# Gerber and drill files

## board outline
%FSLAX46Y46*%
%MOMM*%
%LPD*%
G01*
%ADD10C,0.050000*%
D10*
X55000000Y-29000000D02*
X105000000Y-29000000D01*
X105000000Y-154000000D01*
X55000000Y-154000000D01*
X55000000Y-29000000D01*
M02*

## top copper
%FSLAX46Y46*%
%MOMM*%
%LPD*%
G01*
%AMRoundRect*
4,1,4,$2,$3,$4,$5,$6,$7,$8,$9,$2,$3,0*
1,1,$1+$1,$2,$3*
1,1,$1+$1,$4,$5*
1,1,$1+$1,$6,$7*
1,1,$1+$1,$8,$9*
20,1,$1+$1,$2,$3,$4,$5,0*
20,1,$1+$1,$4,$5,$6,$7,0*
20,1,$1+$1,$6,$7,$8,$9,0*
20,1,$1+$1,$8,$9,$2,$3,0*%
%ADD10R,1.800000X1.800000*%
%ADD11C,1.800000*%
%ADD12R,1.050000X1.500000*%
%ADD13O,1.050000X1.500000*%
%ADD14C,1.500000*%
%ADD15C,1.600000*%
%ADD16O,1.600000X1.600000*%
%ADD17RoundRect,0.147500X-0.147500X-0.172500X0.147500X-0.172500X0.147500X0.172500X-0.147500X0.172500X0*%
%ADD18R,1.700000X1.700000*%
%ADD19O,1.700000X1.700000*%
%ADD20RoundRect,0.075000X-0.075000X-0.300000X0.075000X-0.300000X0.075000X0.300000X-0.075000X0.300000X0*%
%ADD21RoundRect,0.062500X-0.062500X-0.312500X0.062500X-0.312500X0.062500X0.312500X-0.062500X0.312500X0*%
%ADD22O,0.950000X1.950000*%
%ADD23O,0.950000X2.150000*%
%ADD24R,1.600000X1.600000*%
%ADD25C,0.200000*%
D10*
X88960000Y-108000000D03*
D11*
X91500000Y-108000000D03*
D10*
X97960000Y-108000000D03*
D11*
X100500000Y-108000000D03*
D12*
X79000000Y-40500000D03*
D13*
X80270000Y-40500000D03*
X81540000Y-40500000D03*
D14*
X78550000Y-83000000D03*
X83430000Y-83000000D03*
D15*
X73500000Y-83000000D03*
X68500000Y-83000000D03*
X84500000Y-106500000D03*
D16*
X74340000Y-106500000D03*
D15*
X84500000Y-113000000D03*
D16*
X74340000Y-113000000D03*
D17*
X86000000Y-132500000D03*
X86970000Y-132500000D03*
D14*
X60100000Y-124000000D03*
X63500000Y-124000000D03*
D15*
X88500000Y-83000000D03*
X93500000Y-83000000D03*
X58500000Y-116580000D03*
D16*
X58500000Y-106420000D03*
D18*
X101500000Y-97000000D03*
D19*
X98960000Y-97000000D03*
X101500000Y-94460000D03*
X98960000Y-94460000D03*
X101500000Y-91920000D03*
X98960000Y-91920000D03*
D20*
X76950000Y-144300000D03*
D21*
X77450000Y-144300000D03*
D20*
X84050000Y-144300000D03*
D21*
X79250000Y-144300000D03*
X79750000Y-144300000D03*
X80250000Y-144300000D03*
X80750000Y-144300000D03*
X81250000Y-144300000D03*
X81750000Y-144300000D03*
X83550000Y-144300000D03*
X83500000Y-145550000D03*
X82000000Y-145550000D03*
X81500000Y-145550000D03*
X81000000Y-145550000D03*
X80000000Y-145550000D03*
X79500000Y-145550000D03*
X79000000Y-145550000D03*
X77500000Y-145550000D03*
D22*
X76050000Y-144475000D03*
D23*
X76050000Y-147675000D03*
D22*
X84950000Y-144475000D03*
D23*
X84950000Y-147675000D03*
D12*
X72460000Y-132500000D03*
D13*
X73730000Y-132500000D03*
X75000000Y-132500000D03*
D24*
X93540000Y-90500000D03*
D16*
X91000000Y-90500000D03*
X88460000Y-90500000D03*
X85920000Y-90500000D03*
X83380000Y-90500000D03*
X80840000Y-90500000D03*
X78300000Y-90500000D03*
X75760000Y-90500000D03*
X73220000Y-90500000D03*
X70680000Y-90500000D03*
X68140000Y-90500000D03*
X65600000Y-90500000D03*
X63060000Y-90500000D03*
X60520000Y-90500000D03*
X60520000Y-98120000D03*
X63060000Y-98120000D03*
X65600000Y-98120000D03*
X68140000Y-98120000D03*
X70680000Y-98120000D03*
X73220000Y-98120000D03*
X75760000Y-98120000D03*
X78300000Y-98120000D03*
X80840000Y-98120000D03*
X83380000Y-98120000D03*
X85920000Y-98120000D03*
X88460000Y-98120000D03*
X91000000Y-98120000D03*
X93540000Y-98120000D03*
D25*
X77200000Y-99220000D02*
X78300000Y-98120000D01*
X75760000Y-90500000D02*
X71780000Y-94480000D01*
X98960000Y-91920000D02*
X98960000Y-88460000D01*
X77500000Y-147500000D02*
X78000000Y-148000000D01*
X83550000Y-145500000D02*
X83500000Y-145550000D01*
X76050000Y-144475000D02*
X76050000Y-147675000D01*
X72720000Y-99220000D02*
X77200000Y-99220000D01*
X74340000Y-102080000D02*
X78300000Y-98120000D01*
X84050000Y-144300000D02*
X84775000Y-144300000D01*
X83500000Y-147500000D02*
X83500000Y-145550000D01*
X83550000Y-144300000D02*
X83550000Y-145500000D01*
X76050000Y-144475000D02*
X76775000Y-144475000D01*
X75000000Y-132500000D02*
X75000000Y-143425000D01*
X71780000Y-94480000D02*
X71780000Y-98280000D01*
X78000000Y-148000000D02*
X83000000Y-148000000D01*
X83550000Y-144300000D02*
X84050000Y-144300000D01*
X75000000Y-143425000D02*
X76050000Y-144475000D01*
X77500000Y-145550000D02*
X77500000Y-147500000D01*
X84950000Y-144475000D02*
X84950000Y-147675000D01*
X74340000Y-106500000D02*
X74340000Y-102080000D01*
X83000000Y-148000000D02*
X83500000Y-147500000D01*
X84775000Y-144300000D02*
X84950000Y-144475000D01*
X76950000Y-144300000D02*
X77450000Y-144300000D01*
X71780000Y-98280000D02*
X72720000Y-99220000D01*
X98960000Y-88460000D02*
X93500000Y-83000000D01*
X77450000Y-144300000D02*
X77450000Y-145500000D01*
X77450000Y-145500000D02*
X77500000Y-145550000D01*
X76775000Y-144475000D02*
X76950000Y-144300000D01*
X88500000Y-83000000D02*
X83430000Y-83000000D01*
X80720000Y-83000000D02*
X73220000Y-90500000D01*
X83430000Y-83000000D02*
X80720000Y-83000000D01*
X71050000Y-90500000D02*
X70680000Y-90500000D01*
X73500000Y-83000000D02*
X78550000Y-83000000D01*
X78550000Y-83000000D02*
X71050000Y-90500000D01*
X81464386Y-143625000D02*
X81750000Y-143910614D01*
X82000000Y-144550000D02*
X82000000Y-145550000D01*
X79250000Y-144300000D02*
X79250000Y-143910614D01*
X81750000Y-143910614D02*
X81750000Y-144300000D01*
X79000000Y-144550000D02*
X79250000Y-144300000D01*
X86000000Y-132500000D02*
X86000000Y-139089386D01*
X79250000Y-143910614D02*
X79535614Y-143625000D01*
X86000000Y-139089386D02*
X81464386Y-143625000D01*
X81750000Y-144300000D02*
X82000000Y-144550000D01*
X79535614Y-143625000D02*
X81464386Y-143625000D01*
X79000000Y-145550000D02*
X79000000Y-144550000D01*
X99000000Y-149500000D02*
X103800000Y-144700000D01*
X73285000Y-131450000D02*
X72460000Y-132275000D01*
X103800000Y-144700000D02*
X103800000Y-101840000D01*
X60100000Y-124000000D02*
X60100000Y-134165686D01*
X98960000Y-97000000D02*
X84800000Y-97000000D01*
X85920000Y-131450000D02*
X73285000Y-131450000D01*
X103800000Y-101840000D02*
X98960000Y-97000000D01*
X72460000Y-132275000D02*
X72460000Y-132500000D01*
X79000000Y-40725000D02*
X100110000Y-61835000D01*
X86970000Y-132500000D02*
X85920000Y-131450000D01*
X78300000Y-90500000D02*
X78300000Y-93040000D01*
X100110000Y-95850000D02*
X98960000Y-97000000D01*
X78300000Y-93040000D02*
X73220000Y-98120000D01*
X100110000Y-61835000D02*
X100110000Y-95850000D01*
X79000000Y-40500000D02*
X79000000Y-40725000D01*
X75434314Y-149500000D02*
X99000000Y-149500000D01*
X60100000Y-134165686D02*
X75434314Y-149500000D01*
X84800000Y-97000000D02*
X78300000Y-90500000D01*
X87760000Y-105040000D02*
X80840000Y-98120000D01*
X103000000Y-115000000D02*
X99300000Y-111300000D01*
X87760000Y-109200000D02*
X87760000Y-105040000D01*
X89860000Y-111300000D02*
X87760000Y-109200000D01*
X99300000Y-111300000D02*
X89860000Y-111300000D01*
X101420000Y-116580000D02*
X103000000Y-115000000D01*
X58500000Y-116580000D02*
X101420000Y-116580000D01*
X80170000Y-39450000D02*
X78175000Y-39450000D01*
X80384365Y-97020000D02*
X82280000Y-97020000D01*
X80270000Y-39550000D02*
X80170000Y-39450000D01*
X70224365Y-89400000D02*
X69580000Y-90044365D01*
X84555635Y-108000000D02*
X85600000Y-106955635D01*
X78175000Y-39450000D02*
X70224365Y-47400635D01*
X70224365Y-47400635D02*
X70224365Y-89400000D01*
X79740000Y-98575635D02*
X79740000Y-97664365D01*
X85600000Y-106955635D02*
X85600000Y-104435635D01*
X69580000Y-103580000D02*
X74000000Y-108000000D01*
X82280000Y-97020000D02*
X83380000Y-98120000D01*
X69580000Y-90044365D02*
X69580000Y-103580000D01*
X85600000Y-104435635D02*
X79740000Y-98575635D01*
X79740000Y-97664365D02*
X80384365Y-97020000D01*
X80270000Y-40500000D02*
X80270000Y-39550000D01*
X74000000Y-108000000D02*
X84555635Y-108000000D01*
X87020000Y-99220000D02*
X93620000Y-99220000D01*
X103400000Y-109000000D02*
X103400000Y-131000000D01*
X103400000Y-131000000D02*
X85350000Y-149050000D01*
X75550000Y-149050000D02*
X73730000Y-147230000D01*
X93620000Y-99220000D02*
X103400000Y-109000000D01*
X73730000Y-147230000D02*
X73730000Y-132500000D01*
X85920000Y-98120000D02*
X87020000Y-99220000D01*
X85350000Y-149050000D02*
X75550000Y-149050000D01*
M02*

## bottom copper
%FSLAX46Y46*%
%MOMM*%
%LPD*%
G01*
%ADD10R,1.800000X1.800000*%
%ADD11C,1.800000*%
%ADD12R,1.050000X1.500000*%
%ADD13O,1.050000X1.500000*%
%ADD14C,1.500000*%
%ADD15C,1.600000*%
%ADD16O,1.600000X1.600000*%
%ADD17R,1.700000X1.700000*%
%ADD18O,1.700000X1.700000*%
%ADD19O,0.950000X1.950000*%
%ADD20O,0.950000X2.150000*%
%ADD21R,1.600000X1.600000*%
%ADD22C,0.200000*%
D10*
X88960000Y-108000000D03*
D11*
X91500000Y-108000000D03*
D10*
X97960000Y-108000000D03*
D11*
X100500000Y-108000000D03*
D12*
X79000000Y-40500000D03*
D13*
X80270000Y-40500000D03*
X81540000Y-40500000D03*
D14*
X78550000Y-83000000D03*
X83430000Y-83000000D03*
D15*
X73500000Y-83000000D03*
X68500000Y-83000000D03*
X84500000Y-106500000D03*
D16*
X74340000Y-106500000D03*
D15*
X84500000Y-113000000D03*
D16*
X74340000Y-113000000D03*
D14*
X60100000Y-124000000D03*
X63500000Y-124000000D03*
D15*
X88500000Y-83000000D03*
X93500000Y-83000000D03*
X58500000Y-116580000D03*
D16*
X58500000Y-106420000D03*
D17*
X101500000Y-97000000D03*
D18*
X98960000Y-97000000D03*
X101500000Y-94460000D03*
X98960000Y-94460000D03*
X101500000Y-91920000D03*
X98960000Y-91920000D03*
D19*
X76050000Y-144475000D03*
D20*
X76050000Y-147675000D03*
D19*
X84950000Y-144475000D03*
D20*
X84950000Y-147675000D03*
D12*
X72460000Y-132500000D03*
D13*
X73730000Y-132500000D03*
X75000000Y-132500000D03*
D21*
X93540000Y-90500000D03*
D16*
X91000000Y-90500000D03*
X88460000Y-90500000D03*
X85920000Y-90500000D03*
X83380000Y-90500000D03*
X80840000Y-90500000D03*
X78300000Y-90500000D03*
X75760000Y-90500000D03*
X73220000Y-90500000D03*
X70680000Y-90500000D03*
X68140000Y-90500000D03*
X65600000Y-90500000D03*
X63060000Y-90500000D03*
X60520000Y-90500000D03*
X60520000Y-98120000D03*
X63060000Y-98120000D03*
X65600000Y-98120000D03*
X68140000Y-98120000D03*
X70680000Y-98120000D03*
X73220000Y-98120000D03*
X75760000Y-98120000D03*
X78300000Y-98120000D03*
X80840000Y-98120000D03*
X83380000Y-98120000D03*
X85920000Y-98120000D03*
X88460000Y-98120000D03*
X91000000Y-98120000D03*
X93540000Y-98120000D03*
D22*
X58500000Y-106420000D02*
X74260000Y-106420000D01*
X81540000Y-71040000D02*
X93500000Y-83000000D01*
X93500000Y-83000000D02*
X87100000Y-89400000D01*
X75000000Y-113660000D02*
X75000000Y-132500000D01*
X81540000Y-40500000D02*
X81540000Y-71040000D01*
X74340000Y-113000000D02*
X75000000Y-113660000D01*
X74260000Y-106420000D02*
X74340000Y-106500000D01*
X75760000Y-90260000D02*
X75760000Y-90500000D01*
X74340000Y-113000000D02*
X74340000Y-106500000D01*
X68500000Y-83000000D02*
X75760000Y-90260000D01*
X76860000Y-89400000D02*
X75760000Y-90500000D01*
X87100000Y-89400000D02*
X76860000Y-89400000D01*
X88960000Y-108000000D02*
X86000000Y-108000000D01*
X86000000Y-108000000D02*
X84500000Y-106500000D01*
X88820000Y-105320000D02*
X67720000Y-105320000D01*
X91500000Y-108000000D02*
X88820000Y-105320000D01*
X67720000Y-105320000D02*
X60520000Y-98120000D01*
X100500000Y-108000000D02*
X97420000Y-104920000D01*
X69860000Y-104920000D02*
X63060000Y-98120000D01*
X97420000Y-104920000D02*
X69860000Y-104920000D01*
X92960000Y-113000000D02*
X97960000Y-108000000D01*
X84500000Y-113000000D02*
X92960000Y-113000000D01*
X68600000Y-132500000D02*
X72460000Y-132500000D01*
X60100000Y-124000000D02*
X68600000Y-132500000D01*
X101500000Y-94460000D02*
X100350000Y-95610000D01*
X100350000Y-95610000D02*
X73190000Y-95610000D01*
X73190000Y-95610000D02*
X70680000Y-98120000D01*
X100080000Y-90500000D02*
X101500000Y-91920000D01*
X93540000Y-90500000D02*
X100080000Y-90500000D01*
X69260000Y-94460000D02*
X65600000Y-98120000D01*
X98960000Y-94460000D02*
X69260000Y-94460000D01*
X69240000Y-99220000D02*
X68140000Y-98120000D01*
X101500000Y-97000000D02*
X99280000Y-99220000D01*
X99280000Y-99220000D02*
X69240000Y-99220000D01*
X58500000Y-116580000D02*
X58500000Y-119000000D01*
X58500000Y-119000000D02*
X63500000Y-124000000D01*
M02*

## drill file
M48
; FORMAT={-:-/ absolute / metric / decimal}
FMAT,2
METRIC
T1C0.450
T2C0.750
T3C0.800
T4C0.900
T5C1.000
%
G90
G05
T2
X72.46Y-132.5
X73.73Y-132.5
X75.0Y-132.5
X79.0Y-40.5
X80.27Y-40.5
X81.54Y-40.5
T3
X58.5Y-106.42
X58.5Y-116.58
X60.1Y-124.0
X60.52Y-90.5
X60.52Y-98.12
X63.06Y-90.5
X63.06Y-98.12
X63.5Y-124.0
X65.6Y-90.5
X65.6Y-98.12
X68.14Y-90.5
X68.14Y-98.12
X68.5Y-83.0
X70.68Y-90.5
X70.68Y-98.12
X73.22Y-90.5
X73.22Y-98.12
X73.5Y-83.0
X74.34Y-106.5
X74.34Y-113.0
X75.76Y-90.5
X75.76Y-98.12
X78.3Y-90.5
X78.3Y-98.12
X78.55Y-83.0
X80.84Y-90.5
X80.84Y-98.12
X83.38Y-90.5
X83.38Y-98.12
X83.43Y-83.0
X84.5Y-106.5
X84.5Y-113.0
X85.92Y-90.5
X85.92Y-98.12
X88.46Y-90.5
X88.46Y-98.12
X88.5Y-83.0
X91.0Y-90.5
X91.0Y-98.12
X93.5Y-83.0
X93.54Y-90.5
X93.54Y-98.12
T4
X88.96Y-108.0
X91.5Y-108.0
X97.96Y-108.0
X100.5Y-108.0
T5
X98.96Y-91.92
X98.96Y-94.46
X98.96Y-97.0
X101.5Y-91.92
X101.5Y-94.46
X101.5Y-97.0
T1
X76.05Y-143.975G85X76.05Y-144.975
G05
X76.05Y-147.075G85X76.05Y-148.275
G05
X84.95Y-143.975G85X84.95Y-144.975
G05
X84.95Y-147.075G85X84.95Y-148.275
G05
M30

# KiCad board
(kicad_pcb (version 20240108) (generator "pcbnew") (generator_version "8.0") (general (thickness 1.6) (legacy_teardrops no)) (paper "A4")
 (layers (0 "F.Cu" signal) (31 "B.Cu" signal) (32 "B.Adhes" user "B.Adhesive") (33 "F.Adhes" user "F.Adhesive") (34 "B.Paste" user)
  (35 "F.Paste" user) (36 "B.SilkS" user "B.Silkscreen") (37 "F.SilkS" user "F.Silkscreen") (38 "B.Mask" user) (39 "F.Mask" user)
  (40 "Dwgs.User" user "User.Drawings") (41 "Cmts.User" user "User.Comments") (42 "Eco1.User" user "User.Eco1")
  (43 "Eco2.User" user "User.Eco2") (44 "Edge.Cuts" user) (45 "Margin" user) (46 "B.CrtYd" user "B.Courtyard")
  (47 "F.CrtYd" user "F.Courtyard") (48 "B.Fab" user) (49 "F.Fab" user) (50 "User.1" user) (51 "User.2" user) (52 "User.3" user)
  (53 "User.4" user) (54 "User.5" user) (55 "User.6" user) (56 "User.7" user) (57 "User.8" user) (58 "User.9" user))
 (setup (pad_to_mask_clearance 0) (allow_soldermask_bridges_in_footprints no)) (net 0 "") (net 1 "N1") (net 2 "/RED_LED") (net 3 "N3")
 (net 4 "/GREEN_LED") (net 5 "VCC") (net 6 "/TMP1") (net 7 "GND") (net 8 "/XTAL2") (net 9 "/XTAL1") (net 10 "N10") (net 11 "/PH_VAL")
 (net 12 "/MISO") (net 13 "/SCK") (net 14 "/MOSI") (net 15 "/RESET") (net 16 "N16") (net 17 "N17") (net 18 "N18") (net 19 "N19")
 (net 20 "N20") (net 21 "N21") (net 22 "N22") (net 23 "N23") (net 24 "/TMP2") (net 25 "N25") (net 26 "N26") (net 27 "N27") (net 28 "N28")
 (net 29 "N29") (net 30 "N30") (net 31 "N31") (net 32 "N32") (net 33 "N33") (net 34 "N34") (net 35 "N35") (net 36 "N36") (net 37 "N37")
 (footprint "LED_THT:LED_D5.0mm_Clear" (layer "F.Cu") (at 88.96 108)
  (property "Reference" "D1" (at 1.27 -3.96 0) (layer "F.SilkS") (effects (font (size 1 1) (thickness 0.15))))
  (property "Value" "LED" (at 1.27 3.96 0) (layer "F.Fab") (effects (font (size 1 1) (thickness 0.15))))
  (pad "1" thru_hole rect (at 0 0) (size 1.8 1.8) (drill 0.9) (layers "*.Cu" "*.Mask") (remove_unused_layers no) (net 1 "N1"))
  (pad "2" thru_hole circle (at 2.54 0) (size 1.8 1.8) (drill 0.9) (layers "*.Cu" "*.Mask") (remove_unused_layers no) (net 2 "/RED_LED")))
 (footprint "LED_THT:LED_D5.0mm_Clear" (layer "F.Cu") (at 97.96 108)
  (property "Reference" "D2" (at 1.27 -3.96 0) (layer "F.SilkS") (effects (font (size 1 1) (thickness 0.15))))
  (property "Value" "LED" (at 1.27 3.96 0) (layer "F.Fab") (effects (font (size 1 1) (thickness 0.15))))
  (pad "1" thru_hole rect (at 0 0) (size 1.8 1.8) (drill 0.9) (layers "*.Cu" "*.Mask") (remove_unused_layers no) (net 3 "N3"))
  (pad "2" thru_hole circle (at 2.54 0) (size 1.8 1.8) (drill 0.9) (layers "*.Cu" "*.Mask") (remove_unused_layers no) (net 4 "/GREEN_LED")))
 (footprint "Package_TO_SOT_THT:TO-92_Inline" (layer "F.Cu") (at 79 40.5)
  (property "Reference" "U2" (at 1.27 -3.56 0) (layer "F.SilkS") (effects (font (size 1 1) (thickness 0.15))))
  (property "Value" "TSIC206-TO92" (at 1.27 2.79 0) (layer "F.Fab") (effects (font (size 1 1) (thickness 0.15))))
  (pad "1" thru_hole rect (at 0 0) (size 1.05 1.5) (drill 0.75) (layers "*.Cu" "*.Mask") (remove_unused_layers no) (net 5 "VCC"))
  (pad "2" thru_hole oval (at 1.27 0) (size 1.05 1.5) (drill 0.75) (layers "*.Cu" "*.Mask") (remove_unused_layers no) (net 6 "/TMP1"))
  (pad "3" thru_hole oval (at 2.54 0) (size 1.05 1.5) (drill 0.75) (layers "*.Cu" "*.Mask") (remove_unused_layers no) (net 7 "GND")))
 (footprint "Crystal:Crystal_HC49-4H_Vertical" (layer "F.Cu") (at 78.55 83)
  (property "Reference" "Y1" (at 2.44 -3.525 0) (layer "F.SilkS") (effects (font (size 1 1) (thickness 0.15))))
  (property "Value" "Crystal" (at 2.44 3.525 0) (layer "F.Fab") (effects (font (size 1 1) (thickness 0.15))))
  (pad "1" thru_hole circle (at 0 0) (size 1.5 1.5) (drill 0.8) (layers "*.Cu" "*.Mask") (remove_unused_layers no) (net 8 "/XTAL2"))
  (pad "2" thru_hole circle (at 4.88 0) (size 1.5 1.5) (drill 0.8) (layers "*.Cu" "*.Mask") (remove_unused_layers no) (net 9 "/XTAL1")))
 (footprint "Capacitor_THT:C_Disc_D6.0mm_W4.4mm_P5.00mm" (layer "F.Cu") (at 73.5 83 180)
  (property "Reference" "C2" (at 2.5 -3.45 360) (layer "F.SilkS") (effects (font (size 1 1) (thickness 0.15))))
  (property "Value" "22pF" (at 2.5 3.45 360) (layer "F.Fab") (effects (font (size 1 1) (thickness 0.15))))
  (pad "1" thru_hole circle (at 0 0 180) (size 1.6 1.6) (drill 0.8) (layers "*.Cu" "*.Mask") (remove_unused_layers no) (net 8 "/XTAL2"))
  (pad "2" thru_hole circle (at 5 0 180) (size 1.6 1.6) (drill 0.8) (layers "*.Cu" "*.Mask") (remove_unused_layers no) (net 7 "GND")))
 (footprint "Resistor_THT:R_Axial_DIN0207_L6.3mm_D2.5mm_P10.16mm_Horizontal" (layer "F.Cu") (at 84.5 106.5 180)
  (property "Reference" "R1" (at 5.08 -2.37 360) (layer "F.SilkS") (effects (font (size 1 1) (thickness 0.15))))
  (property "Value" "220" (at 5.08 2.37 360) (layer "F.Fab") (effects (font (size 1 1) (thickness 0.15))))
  (pad "1" thru_hole circle (at 0 0 180) (size 1.6 1.6) (drill 0.8) (layers "*.Cu" "*.Mask") (remove_unused_layers no) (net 1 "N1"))
  (pad "2" thru_hole oval (at 10.16 0 180) (size 1.6 1.6) (drill 0.8) (layers "*.Cu" "*.Mask") (remove_unused_layers no) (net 7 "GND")))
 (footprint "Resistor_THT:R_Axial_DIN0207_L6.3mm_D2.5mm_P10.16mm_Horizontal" (layer "F.Cu") (at 84.5 113 180)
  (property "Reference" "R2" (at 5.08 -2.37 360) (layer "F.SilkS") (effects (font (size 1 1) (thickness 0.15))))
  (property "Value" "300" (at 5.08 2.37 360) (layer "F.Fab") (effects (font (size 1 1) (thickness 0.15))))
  (pad "1" thru_hole circle (at 0 0 180) (size 1.6 1.6) (drill 0.8) (layers "*.Cu" "*.Mask") (remove_unused_layers no) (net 3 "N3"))
  (pad "2" thru_hole oval (at 10.16 0 180) (size 1.6 1.6) (drill 0.8) (layers "*.Cu" "*.Mask") (remove_unused_layers no) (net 7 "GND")))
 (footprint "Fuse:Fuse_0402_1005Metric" (layer "F.Cu") (at 86.485 132.5)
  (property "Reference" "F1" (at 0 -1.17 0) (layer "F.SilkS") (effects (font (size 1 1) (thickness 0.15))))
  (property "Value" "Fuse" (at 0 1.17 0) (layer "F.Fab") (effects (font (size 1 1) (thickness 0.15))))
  (pad "1" smd roundrect (at -0.485 0) (size 0.59 0.64) (layers "F.Cu" "F.Paste" "F.Mask") (roundrect_rratio 0.25) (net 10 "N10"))
  (pad "2" smd roundrect (at 0.485 0) (size 0.59 0.64) (layers "F.Cu" "F.Paste" "F.Mask") (roundrect_rratio 0.25) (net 5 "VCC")))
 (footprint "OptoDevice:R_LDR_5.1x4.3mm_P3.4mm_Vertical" (layer "F.Cu") (at 60.1 124)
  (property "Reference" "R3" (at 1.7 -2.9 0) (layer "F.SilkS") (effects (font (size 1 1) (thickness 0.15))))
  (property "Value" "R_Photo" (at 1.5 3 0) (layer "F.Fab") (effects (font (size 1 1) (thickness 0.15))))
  (pad "1" thru_hole circle (at 0 0) (size 1.5 1.5) (drill 0.8) (layers "*.Cu" "*.Mask") (remove_unused_layers no) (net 5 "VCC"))
  (pad "2" thru_hole circle (at 3.4 0) (size 1.5 1.5) (drill 0.8) (layers "*.Cu" "*.Mask") (remove_unused_layers no) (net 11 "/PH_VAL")))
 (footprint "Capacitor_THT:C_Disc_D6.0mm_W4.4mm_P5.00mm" (layer "F.Cu") (at 88.5 83)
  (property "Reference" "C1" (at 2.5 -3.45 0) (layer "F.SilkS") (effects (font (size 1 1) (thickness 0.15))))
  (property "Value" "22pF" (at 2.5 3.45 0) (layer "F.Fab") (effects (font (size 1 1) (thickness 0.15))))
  (pad "1" thru_hole circle (at 0 0) (size 1.6 1.6) (drill 0.8) (layers "*.Cu" "*.Mask") (remove_unused_layers no) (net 9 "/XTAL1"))
  (pad "2" thru_hole circle (at 5 0) (size 1.6 1.6) (drill 0.8) (layers "*.Cu" "*.Mask") (remove_unused_layers no) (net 7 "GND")))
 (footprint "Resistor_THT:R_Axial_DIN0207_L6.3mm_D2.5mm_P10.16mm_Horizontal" (layer "F.Cu") (at 58.5 116.58 90)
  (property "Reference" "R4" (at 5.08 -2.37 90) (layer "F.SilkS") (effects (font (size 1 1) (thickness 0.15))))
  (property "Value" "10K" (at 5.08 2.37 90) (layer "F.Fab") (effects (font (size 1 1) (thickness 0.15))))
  (pad "1" thru_hole circle (at 0 0 90) (size 1.6 1.6) (drill 0.8) (layers "*.Cu" "*.Mask") (remove_unused_layers no) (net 11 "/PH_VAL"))
  (pad "2" thru_hole oval (at 10.16 0 90) (size 1.6 1.6) (drill 0.8) (layers "*.Cu" "*.Mask") (remove_unused_layers no) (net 7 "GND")))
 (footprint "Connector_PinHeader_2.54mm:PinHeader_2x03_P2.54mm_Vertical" (layer "F.Cu") (at 101.5 97 180)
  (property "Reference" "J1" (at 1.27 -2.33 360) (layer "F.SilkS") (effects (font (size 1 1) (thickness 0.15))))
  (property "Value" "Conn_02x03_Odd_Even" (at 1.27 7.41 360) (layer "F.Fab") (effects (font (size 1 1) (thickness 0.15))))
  (pad "1" thru_hole rect (at 0 0 180) (size 1.7 1.7) (drill 1) (layers "*.Cu" "*.Mask") (remove_unused_layers no) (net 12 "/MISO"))
  (pad "2" thru_hole oval (at 2.54 0 180) (size 1.7 1.7) (drill 1) (layers "*.Cu" "*.Mask") (remove_unused_layers no) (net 5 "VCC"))
  (pad "3" thru_hole oval (at 0 2.54 180) (size 1.7 1.7) (drill 1) (layers "*.Cu" "*.Mask") (remove_unused_layers no) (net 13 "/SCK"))
  (pad "4" thru_hole oval (at 2.54 2.54 180) (size 1.7 1.7) (drill 1) (layers "*.Cu" "*.Mask") (remove_unused_layers no) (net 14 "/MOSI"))
  (pad "5" thru_hole oval (at 0 5.08 180) (size 1.7 1.7) (drill 1) (layers "*.Cu" "*.Mask") (remove_unused_layers no) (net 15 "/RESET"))
  (pad "6" thru_hole oval (at 2.54 5.08 180) (size 1.7 1.7) (drill 1) (layers "*.Cu" "*.Mask") (remove_unused_layers no) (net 7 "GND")))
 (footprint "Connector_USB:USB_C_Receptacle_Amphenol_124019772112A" (layer "F.Cu") (at 80.5 147.5)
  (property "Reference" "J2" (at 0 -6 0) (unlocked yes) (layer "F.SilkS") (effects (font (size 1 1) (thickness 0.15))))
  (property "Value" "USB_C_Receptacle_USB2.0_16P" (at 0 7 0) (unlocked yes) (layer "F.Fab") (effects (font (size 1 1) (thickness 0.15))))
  (pad "A1" smd roundrect (at -3.55 -3.2) (size 0.3 0.75) (layers "F.Cu" "F.Paste" "F.Mask") (roundrect_rratio 0.25) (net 7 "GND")
   (thermal_bridge_angle 45))
  (pad "A1" smd roundrect (at -3.05 -3.2) (size 0.25 0.75) (layers "F.Cu" "F.Paste" "F.Mask") (roundrect_rratio 0.25) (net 7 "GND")
   (thermal_bridge_angle 45))
  (pad "A1" smd roundrect (at 3.55 -3.2) (size 0.3 0.75) (layers "F.Cu" "F.Paste" "F.Mask") (roundrect_rratio 0.25) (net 7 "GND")
   (thermal_bridge_angle 45))
  (pad "A4" smd roundrect (at -1.25 -3.2) (size 0.25 0.75) (layers "F.Cu" "F.Paste" "F.Mask") (roundrect_rratio 0.25) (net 10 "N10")
   (thermal_bridge_angle 45))
  (pad "A5" smd roundrect (at -0.75 -3.2) (size 0.25 0.75) (layers "F.Cu" "F.Paste" "F.Mask") (roundrect_rratio 0.25) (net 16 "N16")
   (thermal_bridge_angle 45))
  (pad "A6" smd roundrect (at -0.25 -3.2) (size 0.25 0.75) (layers "F.Cu" "F.Paste" "F.Mask") (roundrect_rratio 0.25) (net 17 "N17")
   (thermal_bridge_angle 45))
  (pad "A7" smd roundrect (at 0.25 -3.2) (size 0.25 0.75) (layers "F.Cu" "F.Paste" "F.Mask") (roundrect_rratio 0.25) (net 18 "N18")
   (thermal_bridge_angle 45))
  (pad "A8" smd roundrect (at 0.75 -3.2) (size 0.25 0.75) (layers "F.Cu" "F.Paste" "F.Mask") (roundrect_rratio 0.25) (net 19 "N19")
   (thermal_bridge_angle 45))
  (pad "A9" smd roundrect (at 1.25 -3.2) (size 0.25 0.75) (layers "F.Cu" "F.Paste" "F.Mask") (roundrect_rratio 0.25) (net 10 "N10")
   (thermal_bridge_angle 45))
  (pad "A12" smd roundrect (at 3.05 -3.2) (size 0.25 0.75) (layers "F.Cu" "F.Paste" "F.Mask") (roundrect_rratio 0.25) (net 7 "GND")
   (thermal_bridge_angle 45))
  (pad "B1" smd roundrect (at 3 -1.95) (size 0.25 0.75) (layers "F.Cu" "F.Paste" "F.Mask") (roundrect_rratio 0.25) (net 7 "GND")
   (thermal_bridge_angle 45))
  (pad "B4" smd roundrect (at 1.5 -1.95) (size 0.25 0.75) (layers "F.Cu" "F.Paste" "F.Mask") (roundrect_rratio 0.25) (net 10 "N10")
   (thermal_bridge_angle 45))
  (pad "B5" smd roundrect (at 1 -1.95) (size 0.25 0.75) (layers "F.Cu" "F.Paste" "F.Mask") (roundrect_rratio 0.25) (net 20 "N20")
   (thermal_bridge_angle 45))
  (pad "B6" smd roundrect (at 0.5 -1.95) (size 0.25 0.75) (layers "F.Cu" "F.Paste" "F.Mask") (roundrect_rratio 0.25) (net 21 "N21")
   (thermal_bridge_angle 45))
  (pad "B7" smd roundrect (at -0.5 -1.95) (size 0.25 0.75) (layers "F.Cu" "F.Paste" "F.Mask") (roundrect_rratio 0.25) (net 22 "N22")
   (thermal_bridge_angle 45))
  (pad "B8" smd roundrect (at -1 -1.95) (size 0.25 0.75) (layers "F.Cu" "F.Paste" "F.Mask") (roundrect_rratio 0.25) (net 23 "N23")
   (thermal_bridge_angle 45))
  (pad "B9" smd roundrect (at -1.5 -1.95) (size 0.25 0.75) (layers "F.Cu" "F.Paste" "F.Mask") (roundrect_rratio 0.25) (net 10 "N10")
   (thermal_bridge_angle 45))
  (pad "B12" smd roundrect (at -3 -1.95) (size 0.25 0.75) (layers "F.Cu" "F.Paste" "F.Mask") (roundrect_rratio 0.25) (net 7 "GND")
   (thermal_bridge_angle 45))
  (pad "S1" thru_hole oval (at -4.45 -3.025) (size 0.95 1.95) (drill oval 0.45 1.45) (layers "*.Cu" "*.Mask") (remove_unused_layers no)
   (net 7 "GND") (thermal_bridge_angle 45))
  (pad "S1" thru_hole oval (at -4.45 0.175) (size 0.95 2.15) (drill oval 0.45 1.65) (layers "*.Cu" "*.Mask") (remove_unused_layers no)
   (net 7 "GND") (thermal_bridge_angle 45))
  (pad "S1" thru_hole oval (at 4.45 -3.025) (size 0.95 1.95) (drill oval 0.45 1.45) (layers "*.Cu" "*.Mask") (remove_unused_layers no)
   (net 7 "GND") (thermal_bridge_angle 45))
  (pad "S1" thru_hole oval (at 4.45 0.175) (size 0.95 2.15) (drill oval 0.45 1.65) (layers "*.Cu" "*.Mask") (remove_unused_layers no)
   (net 7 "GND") (thermal_bridge_angle 45)))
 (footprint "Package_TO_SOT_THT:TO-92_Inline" (layer "F.Cu") (at 72.46 132.5)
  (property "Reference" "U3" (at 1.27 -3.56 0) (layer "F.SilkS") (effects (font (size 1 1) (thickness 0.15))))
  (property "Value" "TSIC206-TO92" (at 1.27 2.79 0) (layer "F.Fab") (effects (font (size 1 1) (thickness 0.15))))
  (pad "1" thru_hole rect (at 0 0) (size 1.05 1.5) (drill 0.75) (layers "*.Cu" "*.Mask") (remove_unused_layers no) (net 5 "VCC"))
  (pad "2" thru_hole oval (at 1.27 0) (size 1.05 1.5) (drill 0.75) (layers "*.Cu" "*.Mask") (remove_unused_layers no) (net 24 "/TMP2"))
  (pad "3" thru_hole oval (at 2.54 0) (size 1.05 1.5) (drill 0.75) (layers "*.Cu" "*.Mask") (remove_unused_layers no) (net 7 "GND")))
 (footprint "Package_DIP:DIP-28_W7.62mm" (layer "F.Cu") (at 93.54 90.5 -90)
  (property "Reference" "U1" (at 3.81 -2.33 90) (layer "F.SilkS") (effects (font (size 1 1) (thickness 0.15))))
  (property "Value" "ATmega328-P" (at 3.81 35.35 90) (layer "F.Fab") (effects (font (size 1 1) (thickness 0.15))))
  (pad "1" thru_hole rect (at 0 0 270) (size 1.6 1.6) (drill 0.8) (layers "*.Cu" "*.Mask") (remove_unused_layers no) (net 15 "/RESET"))
  (pad "2" thru_hole oval (at 0 2.54 270) (size 1.6 1.6) (drill 0.8) (layers "*.Cu" "*.Mask") (remove_unused_layers no) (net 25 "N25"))
  (pad "3" thru_hole oval (at 0 5.08 270) (size 1.6 1.6) (drill 0.8) (layers "*.Cu" "*.Mask") (remove_unused_layers no) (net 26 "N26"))
  (pad "4" thru_hole oval (at 0 7.62 270) (size 1.6 1.6) (drill 0.8) (layers "*.Cu" "*.Mask") (remove_unused_layers no) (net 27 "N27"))
  (pad "5" thru_hole oval (at 0 10.16 270) (size 1.6 1.6) (drill 0.8) (layers "*.Cu" "*.Mask") (remove_unused_layers no) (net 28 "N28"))
  (pad "6" thru_hole oval (at 0 12.7 270) (size 1.6 1.6) (drill 0.8) (layers "*.Cu" "*.Mask") (remove_unused_layers no) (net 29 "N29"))
  (pad "7" thru_hole oval (at 0 15.24 270) (size 1.6 1.6) (drill 0.8) (layers "*.Cu" "*.Mask") (remove_unused_layers no) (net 5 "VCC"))
  (pad "8" thru_hole oval (at 0 17.78 270) (size 1.6 1.6) (drill 0.8) (layers "*.Cu" "*.Mask") (remove_unused_layers no) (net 7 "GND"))
  (pad "9" thru_hole oval (at 0 20.32 270) (size 1.6 1.6) (drill 0.8) (layers "*.Cu" "*.Mask") (remove_unused_layers no) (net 9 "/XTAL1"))
  (pad "10" thru_hole oval (at 0 22.86 270) (size 1.6 1.6) (drill 0.8) (layers "*.Cu" "*.Mask") (remove_unused_layers no) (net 8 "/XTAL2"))
  (pad "11" thru_hole oval (at 0 25.4 270) (size 1.6 1.6) (drill 0.8) (layers "*.Cu" "*.Mask") (remove_unused_layers no) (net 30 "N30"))
  (pad "12" thru_hole oval (at 0 27.94 270) (size 1.6 1.6) (drill 0.8) (layers "*.Cu" "*.Mask") (remove_unused_layers no) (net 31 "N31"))
  (pad "13" thru_hole oval (at 0 30.48 270) (size 1.6 1.6) (drill 0.8) (layers "*.Cu" "*.Mask") (remove_unused_layers no) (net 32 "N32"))
  (pad "14" thru_hole oval (at 0 33.02 270) (size 1.6 1.6) (drill 0.8) (layers "*.Cu" "*.Mask") (remove_unused_layers no) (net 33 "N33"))
  (pad "15" thru_hole oval (at 7.62 33.02 270) (size 1.6 1.6) (drill 0.8) (layers "*.Cu" "*.Mask") (remove_unused_layers no)
   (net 2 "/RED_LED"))
  (pad "16" thru_hole oval (at 7.62 30.48 270) (size 1.6 1.6) (drill 0.8) (layers "*.Cu" "*.Mask") (remove_unused_layers no)
   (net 4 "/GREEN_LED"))
  (pad "17" thru_hole oval (at 7.62 27.94 270) (size 1.6 1.6) (drill 0.8) (layers "*.Cu" "*.Mask") (remove_unused_layers no)
   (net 14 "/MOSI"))
  (pad "18" thru_hole oval (at 7.62 25.4 270) (size 1.6 1.6) (drill 0.8) (layers "*.Cu" "*.Mask") (remove_unused_layers no) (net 12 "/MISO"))
  (pad "19" thru_hole oval (at 7.62 22.86 270) (size 1.6 1.6) (drill 0.8) (layers "*.Cu" "*.Mask") (remove_unused_layers no) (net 13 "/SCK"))
  (pad "20" thru_hole oval (at 7.62 20.32 270) (size 1.6 1.6) (drill 0.8) (layers "*.Cu" "*.Mask") (remove_unused_layers no) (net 5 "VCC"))
  (pad "21" thru_hole oval (at 7.62 17.78 270) (size 1.6 1.6) (drill 0.8) (layers "*.Cu" "*.Mask") (remove_unused_layers no) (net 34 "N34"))
  (pad "22" thru_hole oval (at 7.62 15.24 270) (size 1.6 1.6) (drill 0.8) (layers "*.Cu" "*.Mask") (remove_unused_layers no) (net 7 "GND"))
  (pad "23" thru_hole oval (at 7.62 12.7 270) (size 1.6 1.6) (drill 0.8) (layers "*.Cu" "*.Mask") (remove_unused_layers no)
   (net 11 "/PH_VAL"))
  (pad "24" thru_hole oval (at 7.62 10.16 270) (size 1.6 1.6) (drill 0.8) (layers "*.Cu" "*.Mask") (remove_unused_layers no) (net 6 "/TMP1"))
  (pad "25" thru_hole oval (at 7.62 7.62 270) (size 1.6 1.6) (drill 0.8) (layers "*.Cu" "*.Mask") (remove_unused_layers no) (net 24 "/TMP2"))
  (pad "26" thru_hole oval (at 7.62 5.08 270) (size 1.6 1.6) (drill 0.8) (layers "*.Cu" "*.Mask") (remove_unused_layers no) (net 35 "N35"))
  (pad "27" thru_hole oval (at 7.62 2.54 270) (size 1.6 1.6) (drill 0.8) (layers "*.Cu" "*.Mask") (remove_unused_layers no) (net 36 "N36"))
  (pad "28" thru_hole oval (at 7.62 0 270) (size 1.6 1.6) (drill 0.8) (layers "*.Cu" "*.Mask") (remove_unused_layers no) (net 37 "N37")))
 (gr_rect (start 55 29) (end 105 154) (stroke (width 0.05) (type default)) (fill none) (layer "Edge.Cuts"))
 (segment (start 77.2 99.22) (end 78.3 98.12) (width 0.2) (layer "F.Cu") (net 7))
 (segment (start 75.76 90.5) (end 71.78 94.48) (width 0.2) (layer "F.Cu") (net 7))
 (segment (start 98.96 91.92) (end 98.96 88.46) (width 0.2) (layer "F.Cu") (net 7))
 (segment (start 77.5 147.5) (end 78 148) (width 0.2) (layer "F.Cu") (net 7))
 (segment (start 83.55 145.5) (end 83.5 145.55) (width 0.2) (layer "F.Cu") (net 7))
 (segment (start 76.05 144.475) (end 76.05 147.675) (width 0.2) (layer "F.Cu") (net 7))
 (segment (start 72.72 99.22) (end 77.2 99.22) (width 0.2) (layer "F.Cu") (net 7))
 (segment (start 74.34 102.08) (end 78.3 98.12) (width 0.2) (layer "F.Cu") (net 7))
 (segment (start 84.05 144.3) (end 84.775 144.3) (width 0.2) (layer "F.Cu") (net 7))
 (segment (start 83.5 147.5) (end 83.5 145.55) (width 0.2) (layer "F.Cu") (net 7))
 (segment (start 83.55 144.3) (end 83.55 145.5) (width 0.2) (layer "F.Cu") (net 7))
 (segment (start 76.05 144.475) (end 76.775 144.475) (width 0.2) (layer "F.Cu") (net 7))
 (segment (start 75 132.5) (end 75 143.425) (width 0.2) (layer "F.Cu") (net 7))
 (segment (start 71.78 94.48) (end 71.78 98.28) (width 0.2) (layer "F.Cu") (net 7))
 (segment (start 78 148) (end 83 148) (width 0.2) (layer "F.Cu") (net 7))
 (segment (start 83.55 144.3) (end 84.05 144.3) (width 0.2) (layer "F.Cu") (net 7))
 (segment (start 75 143.425) (end 76.05 144.475) (width 0.2) (layer "F.Cu") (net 7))
 (segment (start 77.5 145.55) (end 77.5 147.5) (width 0.2) (layer "F.Cu") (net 7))
 (segment (start 84.95 144.475) (end 84.95 147.675) (width 0.2) (layer "F.Cu") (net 7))
 (segment (start 74.34 106.5) (end 74.34 102.08) (width 0.2) (layer "F.Cu") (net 7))
 (segment (start 83 148) (end 83.5 147.5) (width 0.2) (layer "F.Cu") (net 7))
 (segment (start 84.775 144.3) (end 84.95 144.475) (width 0.2) (layer "F.Cu") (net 7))
 (segment (start 76.95 144.3) (end 77.45 144.3) (width 0.2) (layer "F.Cu") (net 7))
 (segment (start 71.78 98.28) (end 72.72 99.22) (width 0.2) (layer "F.Cu") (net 7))
 (segment (start 98.96 88.46) (end 93.5 83) (width 0.2) (layer "F.Cu") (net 7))
 (segment (start 77.45 144.3) (end 77.45 145.5) (width 0.2) (layer "F.Cu") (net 7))
 (segment (start 77.45 145.5) (end 77.5 145.55) (width 0.2) (layer "F.Cu") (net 7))
 (segment (start 76.775 144.475) (end 76.95 144.3) (width 0.2) (layer "F.Cu") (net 7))
 (segment (start 58.5 106.42) (end 74.26 106.42) (width 0.2) (layer "B.Cu") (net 7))
 (segment (start 81.54 71.04) (end 93.5 83) (width 0.2) (layer "B.Cu") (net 7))
 (segment (start 93.5 83) (end 87.1 89.4) (width 0.2) (layer "B.Cu") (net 7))
 (segment (start 75 113.66) (end 75 132.5) (width 0.2) (layer "B.Cu") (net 7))
 (segment (start 81.54 40.5) (end 81.54 71.04) (width 0.2) (layer "B.Cu") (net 7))
 (segment (start 74.34 113) (end 75 113.66) (width 0.2) (layer "B.Cu") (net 7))
 (segment (start 74.26 106.42) (end 74.34 106.5) (width 0.2) (layer "B.Cu") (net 7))
 (segment (start 75.76 90.26) (end 75.76 90.5) (width 0.2) (layer "B.Cu") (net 7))
 (segment (start 74.34 113) (end 74.34 106.5) (width 0.2) (layer "B.Cu") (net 7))
 (segment (start 68.5 83) (end 75.76 90.26) (width 0.2) (layer "B.Cu") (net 7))
 (segment (start 76.86 89.4) (end 75.76 90.5) (width 0.2) (layer "B.Cu") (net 7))
 (segment (start 87.1 89.4) (end 76.86 89.4) (width 0.2) (layer "B.Cu") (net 7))
 (segment (start 88.5 83) (end 83.43 83) (width 0.2) (layer "F.Cu") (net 9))
 (segment (start 80.72 83) (end 73.22 90.5) (width 0.2) (layer "F.Cu") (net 9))
 (segment (start 83.43 83) (end 80.72 83) (width 0.2) (layer "F.Cu") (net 9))
 (segment (start 71.05 90.5) (end 70.68 90.5) (width 0.2) (layer "F.Cu") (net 8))
 (segment (start 73.5 83) (end 78.55 83) (width 0.2) (layer "F.Cu") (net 8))
 (segment (start 78.55 83) (end 71.05 90.5) (width 0.2) (layer "F.Cu") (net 8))
 (segment (start 88.96 108) (end 86 108) (width 0.2) (layer "B.Cu") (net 1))
 (segment (start 86 108) (end 84.5 106.5) (width 0.2) (layer "B.Cu") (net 1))
 (segment (start 88.82 105.32) (end 67.72 105.32) (width 0.2) (layer "B.Cu") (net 2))
 (segment (start 91.5 108) (end 88.82 105.32) (width 0.2) (layer "B.Cu") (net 2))
 (segment (start 67.72 105.32) (end 60.52 98.12) (width 0.2) (layer "B.Cu") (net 2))
 (segment (start 100.5 108) (end 97.42 104.92) (width 0.2) (layer "B.Cu") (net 4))
 (segment (start 69.86 104.92) (end 63.06 98.12) (width 0.2) (layer "B.Cu") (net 4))
 (segment (start 97.42 104.92) (end 69.86 104.92) (width 0.2) (layer "B.Cu") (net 4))
 (segment (start 92.96 113) (end 97.96 108) (width 0.2) (layer "B.Cu") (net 3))
 (segment (start 84.5 113) (end 92.96 113) (width 0.2) (layer "B.Cu") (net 3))
 (segment (start 81.464386 143.625) (end 81.75 143.910614) (width 0.2) (layer "F.Cu") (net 10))
 (segment (start 82 144.55) (end 82 145.55) (width 0.2) (layer "F.Cu") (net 10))
 (segment (start 79.25 144.3) (end 79.25 143.910614) (width 0.2) (layer "F.Cu") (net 10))
 (segment (start 81.75 143.910614) (end 81.75 144.3) (width 0.2) (layer "F.Cu") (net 10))
 (segment (start 79 144.55) (end 79.25 144.3) (width 0.2) (layer "F.Cu") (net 10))
 (segment (start 86 132.5) (end 86 139.089386) (width 0.2) (layer "F.Cu") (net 10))
 (segment (start 79.25 143.910614) (end 79.535614 143.625) (width 0.2) (layer "F.Cu") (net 10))
 (segment (start 86 139.089386) (end 81.464386 143.625) (width 0.2) (layer "F.Cu") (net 10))
 (segment (start 81.75 144.3) (end 82 144.55) (width 0.2) (layer "F.Cu") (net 10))
 (segment (start 79.535614 143.625) (end 81.464386 143.625) (width 0.2) (layer "F.Cu") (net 10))
 (segment (start 79 145.55) (end 79 144.55) (width 0.2) (layer "F.Cu") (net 10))
 (segment (start 99 149.5) (end 103.8 144.7) (width 0.2) (layer "F.Cu") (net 5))
 (segment (start 73.285 131.45) (end 72.46 132.275) (width 0.2) (layer "F.Cu") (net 5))
 (segment (start 103.8 144.7) (end 103.8 101.84) (width 0.2) (layer "F.Cu") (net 5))
 (segment (start 60.1 124) (end 60.1 134.165686) (width 0.2) (layer "F.Cu") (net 5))
 (segment (start 98.96 97) (end 84.8 97) (width 0.2) (layer "F.Cu") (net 5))
 (segment (start 85.92 131.45) (end 73.285 131.45) (width 0.2) (layer "F.Cu") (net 5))
 (segment (start 103.8 101.84) (end 98.96 97) (width 0.2) (layer "F.Cu") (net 5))
 (segment (start 72.46 132.275) (end 72.46 132.5) (width 0.2) (layer "F.Cu") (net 5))
 (segment (start 79 40.725) (end 100.11 61.835) (width 0.2) (layer "F.Cu") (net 5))
 (segment (start 86.97 132.5) (end 85.92 131.45) (width 0.2) (layer "F.Cu") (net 5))
 (segment (start 78.3 90.5) (end 78.3 93.04) (width 0.2) (layer "F.Cu") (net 5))
 (segment (start 100.11 95.85) (end 98.96 97) (width 0.2) (layer "F.Cu") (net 5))
 (segment (start 78.3 93.04) (end 73.22 98.12) (width 0.2) (layer "F.Cu") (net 5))
 (segment (start 100.11 61.835) (end 100.11 95.85) (width 0.2) (layer "F.Cu") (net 5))
 (segment (start 79 40.5) (end 79 40.725) (width 0.2) (layer "F.Cu") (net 5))
 (segment (start 75.434314 149.5) (end 99 149.5) (width 0.2) (layer "F.Cu") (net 5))
 (segment (start 60.1 134.165686) (end 75.434314 149.5) (width 0.2) (layer "F.Cu") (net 5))
 (segment (start 84.8 97) (end 78.3 90.5) (width 0.2) (layer "F.Cu") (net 5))
 (segment (start 68.6 132.5) (end 72.46 132.5) (width 0.2) (layer "B.Cu") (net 5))
 (segment (start 60.1 124) (end 68.6 132.5) (width 0.2) (layer "B.Cu") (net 5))
 (segment (start 101.5 94.46) (end 100.35 95.61) (width 0.2) (layer "B.Cu") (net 13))
 (segment (start 100.35 95.61) (end 73.19 95.61) (width 0.2) (layer "B.Cu") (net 13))
 (segment (start 73.19 95.61) (end 70.68 98.12) (width 0.2) (layer "B.Cu") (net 13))
 (segment (start 100.08 90.5) (end 101.5 91.92) (width 0.2) (layer "B.Cu") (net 15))
 (segment (start 93.54 90.5) (end 100.08 90.5) (width 0.2) (layer "B.Cu") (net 15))
 (segment (start 69.26 94.46) (end 65.6 98.12) (width 0.2) (layer "B.Cu") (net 14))
 (segment (start 98.96 94.46) (end 69.26 94.46) (width 0.2) (layer "B.Cu") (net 14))
 (segment (start 69.24 99.22) (end 68.14 98.12) (width 0.2) (layer "B.Cu") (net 12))
 (segment (start 101.5 97) (end 99.28 99.22) (width 0.2) (layer "B.Cu") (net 12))
 (segment (start 99.28 99.22) (end 69.24 99.22) (width 0.2) (layer "B.Cu") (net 12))
 (segment (start 87.76 105.04) (end 80.84 98.12) (width 0.2) (layer "F.Cu") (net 11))
 (segment (start 103 115) (end 99.3 111.3) (width 0.2) (layer "F.Cu") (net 11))
 (segment (start 87.76 109.2) (end 87.76 105.04) (width 0.2) (layer "F.Cu") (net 11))
 (segment (start 89.86 111.3) (end 87.76 109.2) (width 0.2) (layer "F.Cu") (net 11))
 (segment (start 99.3 111.3) (end 89.86 111.3) (width 0.2) (layer "F.Cu") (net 11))
 (segment (start 101.42 116.58) (end 103 115) (width 0.2) (layer "F.Cu") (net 11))
 (segment (start 58.5 116.58) (end 101.42 116.58) (width 0.2) (layer "F.Cu") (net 11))
 (segment (start 58.5 116.58) (end 58.5 119) (width 0.2) (layer "B.Cu") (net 11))
 (segment (start 58.5 119) (end 63.5 124) (width 0.2) (layer "B.Cu") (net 11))
 (segment (start 80.17 39.45) (end 78.175 39.45) (width 0.2) (layer "F.Cu") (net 6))
 (segment (start 80.384365 97.02) (end 82.28 97.02) (width 0.2) (layer "F.Cu") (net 6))
 (segment (start 80.27 39.55) (end 80.17 39.45) (width 0.2) (layer "F.Cu") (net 6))
 (segment (start 70.224365 89.4) (end 69.58 90.044365) (width 0.2) (layer "F.Cu") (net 6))
 (segment (start 84.555635 108) (end 85.6 106.955635) (width 0.2) (layer "F.Cu") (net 6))
 (segment (start 78.175 39.45) (end 70.224365 47.400635) (width 0.2) (layer "F.Cu") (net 6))
 (segment (start 70.224365 47.400635) (end 70.224365 89.4) (width 0.2) (layer "F.Cu") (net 6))
 (segment (start 79.74 98.575635) (end 79.74 97.664365) (width 0.2) (layer "F.Cu") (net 6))
 (segment (start 85.6 106.955635) (end 85.6 104.435635) (width 0.2) (layer "F.Cu") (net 6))
 (segment (start 69.58 103.58) (end 74 108) (width 0.2) (layer "F.Cu") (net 6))
 (segment (start 82.28 97.02) (end 83.38 98.12) (width 0.2) (layer "F.Cu") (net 6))
 (segment (start 69.58 90.044365) (end 69.58 103.58) (width 0.2) (layer "F.Cu") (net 6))
 (segment (start 85.6 104.435635) (end 79.74 98.575635) (width 0.2) (layer "F.Cu") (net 6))
 (segment (start 79.74 97.664365) (end 80.384365 97.02) (width 0.2) (layer "F.Cu") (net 6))
 (segment (start 80.27 40.5) (end 80.27 39.55) (width 0.2) (layer "F.Cu") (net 6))
 (segment (start 74 108) (end 84.555635 108) (width 0.2) (layer "F.Cu") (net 6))
 (segment (start 87.02 99.22) (end 93.62 99.22) (width 0.2) (layer "F.Cu") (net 24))
 (segment (start 103.4 109) (end 103.4 131) (width 0.2) (layer "F.Cu") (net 24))
 (segment (start 103.4 131) (end 85.35 149.05) (width 0.2) (layer "F.Cu") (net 24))
 (segment (start 75.55 149.05) (end 73.73 147.23) (width 0.2) (layer "F.Cu") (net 24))
 (segment (start 93.62 99.22) (end 103.4 109) (width 0.2) (layer "F.Cu") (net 24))
 (segment (start 73.73 147.23) (end 73.73 132.5) (width 0.2) (layer "F.Cu") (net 24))
 (segment (start 85.92 98.12) (end 87.02 99.22) (width 0.2) (layer "F.Cu") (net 24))
 (segment (start 85.35 149.05) (end 75.55 149.05) (width 0.2) (layer "F.Cu") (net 24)))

